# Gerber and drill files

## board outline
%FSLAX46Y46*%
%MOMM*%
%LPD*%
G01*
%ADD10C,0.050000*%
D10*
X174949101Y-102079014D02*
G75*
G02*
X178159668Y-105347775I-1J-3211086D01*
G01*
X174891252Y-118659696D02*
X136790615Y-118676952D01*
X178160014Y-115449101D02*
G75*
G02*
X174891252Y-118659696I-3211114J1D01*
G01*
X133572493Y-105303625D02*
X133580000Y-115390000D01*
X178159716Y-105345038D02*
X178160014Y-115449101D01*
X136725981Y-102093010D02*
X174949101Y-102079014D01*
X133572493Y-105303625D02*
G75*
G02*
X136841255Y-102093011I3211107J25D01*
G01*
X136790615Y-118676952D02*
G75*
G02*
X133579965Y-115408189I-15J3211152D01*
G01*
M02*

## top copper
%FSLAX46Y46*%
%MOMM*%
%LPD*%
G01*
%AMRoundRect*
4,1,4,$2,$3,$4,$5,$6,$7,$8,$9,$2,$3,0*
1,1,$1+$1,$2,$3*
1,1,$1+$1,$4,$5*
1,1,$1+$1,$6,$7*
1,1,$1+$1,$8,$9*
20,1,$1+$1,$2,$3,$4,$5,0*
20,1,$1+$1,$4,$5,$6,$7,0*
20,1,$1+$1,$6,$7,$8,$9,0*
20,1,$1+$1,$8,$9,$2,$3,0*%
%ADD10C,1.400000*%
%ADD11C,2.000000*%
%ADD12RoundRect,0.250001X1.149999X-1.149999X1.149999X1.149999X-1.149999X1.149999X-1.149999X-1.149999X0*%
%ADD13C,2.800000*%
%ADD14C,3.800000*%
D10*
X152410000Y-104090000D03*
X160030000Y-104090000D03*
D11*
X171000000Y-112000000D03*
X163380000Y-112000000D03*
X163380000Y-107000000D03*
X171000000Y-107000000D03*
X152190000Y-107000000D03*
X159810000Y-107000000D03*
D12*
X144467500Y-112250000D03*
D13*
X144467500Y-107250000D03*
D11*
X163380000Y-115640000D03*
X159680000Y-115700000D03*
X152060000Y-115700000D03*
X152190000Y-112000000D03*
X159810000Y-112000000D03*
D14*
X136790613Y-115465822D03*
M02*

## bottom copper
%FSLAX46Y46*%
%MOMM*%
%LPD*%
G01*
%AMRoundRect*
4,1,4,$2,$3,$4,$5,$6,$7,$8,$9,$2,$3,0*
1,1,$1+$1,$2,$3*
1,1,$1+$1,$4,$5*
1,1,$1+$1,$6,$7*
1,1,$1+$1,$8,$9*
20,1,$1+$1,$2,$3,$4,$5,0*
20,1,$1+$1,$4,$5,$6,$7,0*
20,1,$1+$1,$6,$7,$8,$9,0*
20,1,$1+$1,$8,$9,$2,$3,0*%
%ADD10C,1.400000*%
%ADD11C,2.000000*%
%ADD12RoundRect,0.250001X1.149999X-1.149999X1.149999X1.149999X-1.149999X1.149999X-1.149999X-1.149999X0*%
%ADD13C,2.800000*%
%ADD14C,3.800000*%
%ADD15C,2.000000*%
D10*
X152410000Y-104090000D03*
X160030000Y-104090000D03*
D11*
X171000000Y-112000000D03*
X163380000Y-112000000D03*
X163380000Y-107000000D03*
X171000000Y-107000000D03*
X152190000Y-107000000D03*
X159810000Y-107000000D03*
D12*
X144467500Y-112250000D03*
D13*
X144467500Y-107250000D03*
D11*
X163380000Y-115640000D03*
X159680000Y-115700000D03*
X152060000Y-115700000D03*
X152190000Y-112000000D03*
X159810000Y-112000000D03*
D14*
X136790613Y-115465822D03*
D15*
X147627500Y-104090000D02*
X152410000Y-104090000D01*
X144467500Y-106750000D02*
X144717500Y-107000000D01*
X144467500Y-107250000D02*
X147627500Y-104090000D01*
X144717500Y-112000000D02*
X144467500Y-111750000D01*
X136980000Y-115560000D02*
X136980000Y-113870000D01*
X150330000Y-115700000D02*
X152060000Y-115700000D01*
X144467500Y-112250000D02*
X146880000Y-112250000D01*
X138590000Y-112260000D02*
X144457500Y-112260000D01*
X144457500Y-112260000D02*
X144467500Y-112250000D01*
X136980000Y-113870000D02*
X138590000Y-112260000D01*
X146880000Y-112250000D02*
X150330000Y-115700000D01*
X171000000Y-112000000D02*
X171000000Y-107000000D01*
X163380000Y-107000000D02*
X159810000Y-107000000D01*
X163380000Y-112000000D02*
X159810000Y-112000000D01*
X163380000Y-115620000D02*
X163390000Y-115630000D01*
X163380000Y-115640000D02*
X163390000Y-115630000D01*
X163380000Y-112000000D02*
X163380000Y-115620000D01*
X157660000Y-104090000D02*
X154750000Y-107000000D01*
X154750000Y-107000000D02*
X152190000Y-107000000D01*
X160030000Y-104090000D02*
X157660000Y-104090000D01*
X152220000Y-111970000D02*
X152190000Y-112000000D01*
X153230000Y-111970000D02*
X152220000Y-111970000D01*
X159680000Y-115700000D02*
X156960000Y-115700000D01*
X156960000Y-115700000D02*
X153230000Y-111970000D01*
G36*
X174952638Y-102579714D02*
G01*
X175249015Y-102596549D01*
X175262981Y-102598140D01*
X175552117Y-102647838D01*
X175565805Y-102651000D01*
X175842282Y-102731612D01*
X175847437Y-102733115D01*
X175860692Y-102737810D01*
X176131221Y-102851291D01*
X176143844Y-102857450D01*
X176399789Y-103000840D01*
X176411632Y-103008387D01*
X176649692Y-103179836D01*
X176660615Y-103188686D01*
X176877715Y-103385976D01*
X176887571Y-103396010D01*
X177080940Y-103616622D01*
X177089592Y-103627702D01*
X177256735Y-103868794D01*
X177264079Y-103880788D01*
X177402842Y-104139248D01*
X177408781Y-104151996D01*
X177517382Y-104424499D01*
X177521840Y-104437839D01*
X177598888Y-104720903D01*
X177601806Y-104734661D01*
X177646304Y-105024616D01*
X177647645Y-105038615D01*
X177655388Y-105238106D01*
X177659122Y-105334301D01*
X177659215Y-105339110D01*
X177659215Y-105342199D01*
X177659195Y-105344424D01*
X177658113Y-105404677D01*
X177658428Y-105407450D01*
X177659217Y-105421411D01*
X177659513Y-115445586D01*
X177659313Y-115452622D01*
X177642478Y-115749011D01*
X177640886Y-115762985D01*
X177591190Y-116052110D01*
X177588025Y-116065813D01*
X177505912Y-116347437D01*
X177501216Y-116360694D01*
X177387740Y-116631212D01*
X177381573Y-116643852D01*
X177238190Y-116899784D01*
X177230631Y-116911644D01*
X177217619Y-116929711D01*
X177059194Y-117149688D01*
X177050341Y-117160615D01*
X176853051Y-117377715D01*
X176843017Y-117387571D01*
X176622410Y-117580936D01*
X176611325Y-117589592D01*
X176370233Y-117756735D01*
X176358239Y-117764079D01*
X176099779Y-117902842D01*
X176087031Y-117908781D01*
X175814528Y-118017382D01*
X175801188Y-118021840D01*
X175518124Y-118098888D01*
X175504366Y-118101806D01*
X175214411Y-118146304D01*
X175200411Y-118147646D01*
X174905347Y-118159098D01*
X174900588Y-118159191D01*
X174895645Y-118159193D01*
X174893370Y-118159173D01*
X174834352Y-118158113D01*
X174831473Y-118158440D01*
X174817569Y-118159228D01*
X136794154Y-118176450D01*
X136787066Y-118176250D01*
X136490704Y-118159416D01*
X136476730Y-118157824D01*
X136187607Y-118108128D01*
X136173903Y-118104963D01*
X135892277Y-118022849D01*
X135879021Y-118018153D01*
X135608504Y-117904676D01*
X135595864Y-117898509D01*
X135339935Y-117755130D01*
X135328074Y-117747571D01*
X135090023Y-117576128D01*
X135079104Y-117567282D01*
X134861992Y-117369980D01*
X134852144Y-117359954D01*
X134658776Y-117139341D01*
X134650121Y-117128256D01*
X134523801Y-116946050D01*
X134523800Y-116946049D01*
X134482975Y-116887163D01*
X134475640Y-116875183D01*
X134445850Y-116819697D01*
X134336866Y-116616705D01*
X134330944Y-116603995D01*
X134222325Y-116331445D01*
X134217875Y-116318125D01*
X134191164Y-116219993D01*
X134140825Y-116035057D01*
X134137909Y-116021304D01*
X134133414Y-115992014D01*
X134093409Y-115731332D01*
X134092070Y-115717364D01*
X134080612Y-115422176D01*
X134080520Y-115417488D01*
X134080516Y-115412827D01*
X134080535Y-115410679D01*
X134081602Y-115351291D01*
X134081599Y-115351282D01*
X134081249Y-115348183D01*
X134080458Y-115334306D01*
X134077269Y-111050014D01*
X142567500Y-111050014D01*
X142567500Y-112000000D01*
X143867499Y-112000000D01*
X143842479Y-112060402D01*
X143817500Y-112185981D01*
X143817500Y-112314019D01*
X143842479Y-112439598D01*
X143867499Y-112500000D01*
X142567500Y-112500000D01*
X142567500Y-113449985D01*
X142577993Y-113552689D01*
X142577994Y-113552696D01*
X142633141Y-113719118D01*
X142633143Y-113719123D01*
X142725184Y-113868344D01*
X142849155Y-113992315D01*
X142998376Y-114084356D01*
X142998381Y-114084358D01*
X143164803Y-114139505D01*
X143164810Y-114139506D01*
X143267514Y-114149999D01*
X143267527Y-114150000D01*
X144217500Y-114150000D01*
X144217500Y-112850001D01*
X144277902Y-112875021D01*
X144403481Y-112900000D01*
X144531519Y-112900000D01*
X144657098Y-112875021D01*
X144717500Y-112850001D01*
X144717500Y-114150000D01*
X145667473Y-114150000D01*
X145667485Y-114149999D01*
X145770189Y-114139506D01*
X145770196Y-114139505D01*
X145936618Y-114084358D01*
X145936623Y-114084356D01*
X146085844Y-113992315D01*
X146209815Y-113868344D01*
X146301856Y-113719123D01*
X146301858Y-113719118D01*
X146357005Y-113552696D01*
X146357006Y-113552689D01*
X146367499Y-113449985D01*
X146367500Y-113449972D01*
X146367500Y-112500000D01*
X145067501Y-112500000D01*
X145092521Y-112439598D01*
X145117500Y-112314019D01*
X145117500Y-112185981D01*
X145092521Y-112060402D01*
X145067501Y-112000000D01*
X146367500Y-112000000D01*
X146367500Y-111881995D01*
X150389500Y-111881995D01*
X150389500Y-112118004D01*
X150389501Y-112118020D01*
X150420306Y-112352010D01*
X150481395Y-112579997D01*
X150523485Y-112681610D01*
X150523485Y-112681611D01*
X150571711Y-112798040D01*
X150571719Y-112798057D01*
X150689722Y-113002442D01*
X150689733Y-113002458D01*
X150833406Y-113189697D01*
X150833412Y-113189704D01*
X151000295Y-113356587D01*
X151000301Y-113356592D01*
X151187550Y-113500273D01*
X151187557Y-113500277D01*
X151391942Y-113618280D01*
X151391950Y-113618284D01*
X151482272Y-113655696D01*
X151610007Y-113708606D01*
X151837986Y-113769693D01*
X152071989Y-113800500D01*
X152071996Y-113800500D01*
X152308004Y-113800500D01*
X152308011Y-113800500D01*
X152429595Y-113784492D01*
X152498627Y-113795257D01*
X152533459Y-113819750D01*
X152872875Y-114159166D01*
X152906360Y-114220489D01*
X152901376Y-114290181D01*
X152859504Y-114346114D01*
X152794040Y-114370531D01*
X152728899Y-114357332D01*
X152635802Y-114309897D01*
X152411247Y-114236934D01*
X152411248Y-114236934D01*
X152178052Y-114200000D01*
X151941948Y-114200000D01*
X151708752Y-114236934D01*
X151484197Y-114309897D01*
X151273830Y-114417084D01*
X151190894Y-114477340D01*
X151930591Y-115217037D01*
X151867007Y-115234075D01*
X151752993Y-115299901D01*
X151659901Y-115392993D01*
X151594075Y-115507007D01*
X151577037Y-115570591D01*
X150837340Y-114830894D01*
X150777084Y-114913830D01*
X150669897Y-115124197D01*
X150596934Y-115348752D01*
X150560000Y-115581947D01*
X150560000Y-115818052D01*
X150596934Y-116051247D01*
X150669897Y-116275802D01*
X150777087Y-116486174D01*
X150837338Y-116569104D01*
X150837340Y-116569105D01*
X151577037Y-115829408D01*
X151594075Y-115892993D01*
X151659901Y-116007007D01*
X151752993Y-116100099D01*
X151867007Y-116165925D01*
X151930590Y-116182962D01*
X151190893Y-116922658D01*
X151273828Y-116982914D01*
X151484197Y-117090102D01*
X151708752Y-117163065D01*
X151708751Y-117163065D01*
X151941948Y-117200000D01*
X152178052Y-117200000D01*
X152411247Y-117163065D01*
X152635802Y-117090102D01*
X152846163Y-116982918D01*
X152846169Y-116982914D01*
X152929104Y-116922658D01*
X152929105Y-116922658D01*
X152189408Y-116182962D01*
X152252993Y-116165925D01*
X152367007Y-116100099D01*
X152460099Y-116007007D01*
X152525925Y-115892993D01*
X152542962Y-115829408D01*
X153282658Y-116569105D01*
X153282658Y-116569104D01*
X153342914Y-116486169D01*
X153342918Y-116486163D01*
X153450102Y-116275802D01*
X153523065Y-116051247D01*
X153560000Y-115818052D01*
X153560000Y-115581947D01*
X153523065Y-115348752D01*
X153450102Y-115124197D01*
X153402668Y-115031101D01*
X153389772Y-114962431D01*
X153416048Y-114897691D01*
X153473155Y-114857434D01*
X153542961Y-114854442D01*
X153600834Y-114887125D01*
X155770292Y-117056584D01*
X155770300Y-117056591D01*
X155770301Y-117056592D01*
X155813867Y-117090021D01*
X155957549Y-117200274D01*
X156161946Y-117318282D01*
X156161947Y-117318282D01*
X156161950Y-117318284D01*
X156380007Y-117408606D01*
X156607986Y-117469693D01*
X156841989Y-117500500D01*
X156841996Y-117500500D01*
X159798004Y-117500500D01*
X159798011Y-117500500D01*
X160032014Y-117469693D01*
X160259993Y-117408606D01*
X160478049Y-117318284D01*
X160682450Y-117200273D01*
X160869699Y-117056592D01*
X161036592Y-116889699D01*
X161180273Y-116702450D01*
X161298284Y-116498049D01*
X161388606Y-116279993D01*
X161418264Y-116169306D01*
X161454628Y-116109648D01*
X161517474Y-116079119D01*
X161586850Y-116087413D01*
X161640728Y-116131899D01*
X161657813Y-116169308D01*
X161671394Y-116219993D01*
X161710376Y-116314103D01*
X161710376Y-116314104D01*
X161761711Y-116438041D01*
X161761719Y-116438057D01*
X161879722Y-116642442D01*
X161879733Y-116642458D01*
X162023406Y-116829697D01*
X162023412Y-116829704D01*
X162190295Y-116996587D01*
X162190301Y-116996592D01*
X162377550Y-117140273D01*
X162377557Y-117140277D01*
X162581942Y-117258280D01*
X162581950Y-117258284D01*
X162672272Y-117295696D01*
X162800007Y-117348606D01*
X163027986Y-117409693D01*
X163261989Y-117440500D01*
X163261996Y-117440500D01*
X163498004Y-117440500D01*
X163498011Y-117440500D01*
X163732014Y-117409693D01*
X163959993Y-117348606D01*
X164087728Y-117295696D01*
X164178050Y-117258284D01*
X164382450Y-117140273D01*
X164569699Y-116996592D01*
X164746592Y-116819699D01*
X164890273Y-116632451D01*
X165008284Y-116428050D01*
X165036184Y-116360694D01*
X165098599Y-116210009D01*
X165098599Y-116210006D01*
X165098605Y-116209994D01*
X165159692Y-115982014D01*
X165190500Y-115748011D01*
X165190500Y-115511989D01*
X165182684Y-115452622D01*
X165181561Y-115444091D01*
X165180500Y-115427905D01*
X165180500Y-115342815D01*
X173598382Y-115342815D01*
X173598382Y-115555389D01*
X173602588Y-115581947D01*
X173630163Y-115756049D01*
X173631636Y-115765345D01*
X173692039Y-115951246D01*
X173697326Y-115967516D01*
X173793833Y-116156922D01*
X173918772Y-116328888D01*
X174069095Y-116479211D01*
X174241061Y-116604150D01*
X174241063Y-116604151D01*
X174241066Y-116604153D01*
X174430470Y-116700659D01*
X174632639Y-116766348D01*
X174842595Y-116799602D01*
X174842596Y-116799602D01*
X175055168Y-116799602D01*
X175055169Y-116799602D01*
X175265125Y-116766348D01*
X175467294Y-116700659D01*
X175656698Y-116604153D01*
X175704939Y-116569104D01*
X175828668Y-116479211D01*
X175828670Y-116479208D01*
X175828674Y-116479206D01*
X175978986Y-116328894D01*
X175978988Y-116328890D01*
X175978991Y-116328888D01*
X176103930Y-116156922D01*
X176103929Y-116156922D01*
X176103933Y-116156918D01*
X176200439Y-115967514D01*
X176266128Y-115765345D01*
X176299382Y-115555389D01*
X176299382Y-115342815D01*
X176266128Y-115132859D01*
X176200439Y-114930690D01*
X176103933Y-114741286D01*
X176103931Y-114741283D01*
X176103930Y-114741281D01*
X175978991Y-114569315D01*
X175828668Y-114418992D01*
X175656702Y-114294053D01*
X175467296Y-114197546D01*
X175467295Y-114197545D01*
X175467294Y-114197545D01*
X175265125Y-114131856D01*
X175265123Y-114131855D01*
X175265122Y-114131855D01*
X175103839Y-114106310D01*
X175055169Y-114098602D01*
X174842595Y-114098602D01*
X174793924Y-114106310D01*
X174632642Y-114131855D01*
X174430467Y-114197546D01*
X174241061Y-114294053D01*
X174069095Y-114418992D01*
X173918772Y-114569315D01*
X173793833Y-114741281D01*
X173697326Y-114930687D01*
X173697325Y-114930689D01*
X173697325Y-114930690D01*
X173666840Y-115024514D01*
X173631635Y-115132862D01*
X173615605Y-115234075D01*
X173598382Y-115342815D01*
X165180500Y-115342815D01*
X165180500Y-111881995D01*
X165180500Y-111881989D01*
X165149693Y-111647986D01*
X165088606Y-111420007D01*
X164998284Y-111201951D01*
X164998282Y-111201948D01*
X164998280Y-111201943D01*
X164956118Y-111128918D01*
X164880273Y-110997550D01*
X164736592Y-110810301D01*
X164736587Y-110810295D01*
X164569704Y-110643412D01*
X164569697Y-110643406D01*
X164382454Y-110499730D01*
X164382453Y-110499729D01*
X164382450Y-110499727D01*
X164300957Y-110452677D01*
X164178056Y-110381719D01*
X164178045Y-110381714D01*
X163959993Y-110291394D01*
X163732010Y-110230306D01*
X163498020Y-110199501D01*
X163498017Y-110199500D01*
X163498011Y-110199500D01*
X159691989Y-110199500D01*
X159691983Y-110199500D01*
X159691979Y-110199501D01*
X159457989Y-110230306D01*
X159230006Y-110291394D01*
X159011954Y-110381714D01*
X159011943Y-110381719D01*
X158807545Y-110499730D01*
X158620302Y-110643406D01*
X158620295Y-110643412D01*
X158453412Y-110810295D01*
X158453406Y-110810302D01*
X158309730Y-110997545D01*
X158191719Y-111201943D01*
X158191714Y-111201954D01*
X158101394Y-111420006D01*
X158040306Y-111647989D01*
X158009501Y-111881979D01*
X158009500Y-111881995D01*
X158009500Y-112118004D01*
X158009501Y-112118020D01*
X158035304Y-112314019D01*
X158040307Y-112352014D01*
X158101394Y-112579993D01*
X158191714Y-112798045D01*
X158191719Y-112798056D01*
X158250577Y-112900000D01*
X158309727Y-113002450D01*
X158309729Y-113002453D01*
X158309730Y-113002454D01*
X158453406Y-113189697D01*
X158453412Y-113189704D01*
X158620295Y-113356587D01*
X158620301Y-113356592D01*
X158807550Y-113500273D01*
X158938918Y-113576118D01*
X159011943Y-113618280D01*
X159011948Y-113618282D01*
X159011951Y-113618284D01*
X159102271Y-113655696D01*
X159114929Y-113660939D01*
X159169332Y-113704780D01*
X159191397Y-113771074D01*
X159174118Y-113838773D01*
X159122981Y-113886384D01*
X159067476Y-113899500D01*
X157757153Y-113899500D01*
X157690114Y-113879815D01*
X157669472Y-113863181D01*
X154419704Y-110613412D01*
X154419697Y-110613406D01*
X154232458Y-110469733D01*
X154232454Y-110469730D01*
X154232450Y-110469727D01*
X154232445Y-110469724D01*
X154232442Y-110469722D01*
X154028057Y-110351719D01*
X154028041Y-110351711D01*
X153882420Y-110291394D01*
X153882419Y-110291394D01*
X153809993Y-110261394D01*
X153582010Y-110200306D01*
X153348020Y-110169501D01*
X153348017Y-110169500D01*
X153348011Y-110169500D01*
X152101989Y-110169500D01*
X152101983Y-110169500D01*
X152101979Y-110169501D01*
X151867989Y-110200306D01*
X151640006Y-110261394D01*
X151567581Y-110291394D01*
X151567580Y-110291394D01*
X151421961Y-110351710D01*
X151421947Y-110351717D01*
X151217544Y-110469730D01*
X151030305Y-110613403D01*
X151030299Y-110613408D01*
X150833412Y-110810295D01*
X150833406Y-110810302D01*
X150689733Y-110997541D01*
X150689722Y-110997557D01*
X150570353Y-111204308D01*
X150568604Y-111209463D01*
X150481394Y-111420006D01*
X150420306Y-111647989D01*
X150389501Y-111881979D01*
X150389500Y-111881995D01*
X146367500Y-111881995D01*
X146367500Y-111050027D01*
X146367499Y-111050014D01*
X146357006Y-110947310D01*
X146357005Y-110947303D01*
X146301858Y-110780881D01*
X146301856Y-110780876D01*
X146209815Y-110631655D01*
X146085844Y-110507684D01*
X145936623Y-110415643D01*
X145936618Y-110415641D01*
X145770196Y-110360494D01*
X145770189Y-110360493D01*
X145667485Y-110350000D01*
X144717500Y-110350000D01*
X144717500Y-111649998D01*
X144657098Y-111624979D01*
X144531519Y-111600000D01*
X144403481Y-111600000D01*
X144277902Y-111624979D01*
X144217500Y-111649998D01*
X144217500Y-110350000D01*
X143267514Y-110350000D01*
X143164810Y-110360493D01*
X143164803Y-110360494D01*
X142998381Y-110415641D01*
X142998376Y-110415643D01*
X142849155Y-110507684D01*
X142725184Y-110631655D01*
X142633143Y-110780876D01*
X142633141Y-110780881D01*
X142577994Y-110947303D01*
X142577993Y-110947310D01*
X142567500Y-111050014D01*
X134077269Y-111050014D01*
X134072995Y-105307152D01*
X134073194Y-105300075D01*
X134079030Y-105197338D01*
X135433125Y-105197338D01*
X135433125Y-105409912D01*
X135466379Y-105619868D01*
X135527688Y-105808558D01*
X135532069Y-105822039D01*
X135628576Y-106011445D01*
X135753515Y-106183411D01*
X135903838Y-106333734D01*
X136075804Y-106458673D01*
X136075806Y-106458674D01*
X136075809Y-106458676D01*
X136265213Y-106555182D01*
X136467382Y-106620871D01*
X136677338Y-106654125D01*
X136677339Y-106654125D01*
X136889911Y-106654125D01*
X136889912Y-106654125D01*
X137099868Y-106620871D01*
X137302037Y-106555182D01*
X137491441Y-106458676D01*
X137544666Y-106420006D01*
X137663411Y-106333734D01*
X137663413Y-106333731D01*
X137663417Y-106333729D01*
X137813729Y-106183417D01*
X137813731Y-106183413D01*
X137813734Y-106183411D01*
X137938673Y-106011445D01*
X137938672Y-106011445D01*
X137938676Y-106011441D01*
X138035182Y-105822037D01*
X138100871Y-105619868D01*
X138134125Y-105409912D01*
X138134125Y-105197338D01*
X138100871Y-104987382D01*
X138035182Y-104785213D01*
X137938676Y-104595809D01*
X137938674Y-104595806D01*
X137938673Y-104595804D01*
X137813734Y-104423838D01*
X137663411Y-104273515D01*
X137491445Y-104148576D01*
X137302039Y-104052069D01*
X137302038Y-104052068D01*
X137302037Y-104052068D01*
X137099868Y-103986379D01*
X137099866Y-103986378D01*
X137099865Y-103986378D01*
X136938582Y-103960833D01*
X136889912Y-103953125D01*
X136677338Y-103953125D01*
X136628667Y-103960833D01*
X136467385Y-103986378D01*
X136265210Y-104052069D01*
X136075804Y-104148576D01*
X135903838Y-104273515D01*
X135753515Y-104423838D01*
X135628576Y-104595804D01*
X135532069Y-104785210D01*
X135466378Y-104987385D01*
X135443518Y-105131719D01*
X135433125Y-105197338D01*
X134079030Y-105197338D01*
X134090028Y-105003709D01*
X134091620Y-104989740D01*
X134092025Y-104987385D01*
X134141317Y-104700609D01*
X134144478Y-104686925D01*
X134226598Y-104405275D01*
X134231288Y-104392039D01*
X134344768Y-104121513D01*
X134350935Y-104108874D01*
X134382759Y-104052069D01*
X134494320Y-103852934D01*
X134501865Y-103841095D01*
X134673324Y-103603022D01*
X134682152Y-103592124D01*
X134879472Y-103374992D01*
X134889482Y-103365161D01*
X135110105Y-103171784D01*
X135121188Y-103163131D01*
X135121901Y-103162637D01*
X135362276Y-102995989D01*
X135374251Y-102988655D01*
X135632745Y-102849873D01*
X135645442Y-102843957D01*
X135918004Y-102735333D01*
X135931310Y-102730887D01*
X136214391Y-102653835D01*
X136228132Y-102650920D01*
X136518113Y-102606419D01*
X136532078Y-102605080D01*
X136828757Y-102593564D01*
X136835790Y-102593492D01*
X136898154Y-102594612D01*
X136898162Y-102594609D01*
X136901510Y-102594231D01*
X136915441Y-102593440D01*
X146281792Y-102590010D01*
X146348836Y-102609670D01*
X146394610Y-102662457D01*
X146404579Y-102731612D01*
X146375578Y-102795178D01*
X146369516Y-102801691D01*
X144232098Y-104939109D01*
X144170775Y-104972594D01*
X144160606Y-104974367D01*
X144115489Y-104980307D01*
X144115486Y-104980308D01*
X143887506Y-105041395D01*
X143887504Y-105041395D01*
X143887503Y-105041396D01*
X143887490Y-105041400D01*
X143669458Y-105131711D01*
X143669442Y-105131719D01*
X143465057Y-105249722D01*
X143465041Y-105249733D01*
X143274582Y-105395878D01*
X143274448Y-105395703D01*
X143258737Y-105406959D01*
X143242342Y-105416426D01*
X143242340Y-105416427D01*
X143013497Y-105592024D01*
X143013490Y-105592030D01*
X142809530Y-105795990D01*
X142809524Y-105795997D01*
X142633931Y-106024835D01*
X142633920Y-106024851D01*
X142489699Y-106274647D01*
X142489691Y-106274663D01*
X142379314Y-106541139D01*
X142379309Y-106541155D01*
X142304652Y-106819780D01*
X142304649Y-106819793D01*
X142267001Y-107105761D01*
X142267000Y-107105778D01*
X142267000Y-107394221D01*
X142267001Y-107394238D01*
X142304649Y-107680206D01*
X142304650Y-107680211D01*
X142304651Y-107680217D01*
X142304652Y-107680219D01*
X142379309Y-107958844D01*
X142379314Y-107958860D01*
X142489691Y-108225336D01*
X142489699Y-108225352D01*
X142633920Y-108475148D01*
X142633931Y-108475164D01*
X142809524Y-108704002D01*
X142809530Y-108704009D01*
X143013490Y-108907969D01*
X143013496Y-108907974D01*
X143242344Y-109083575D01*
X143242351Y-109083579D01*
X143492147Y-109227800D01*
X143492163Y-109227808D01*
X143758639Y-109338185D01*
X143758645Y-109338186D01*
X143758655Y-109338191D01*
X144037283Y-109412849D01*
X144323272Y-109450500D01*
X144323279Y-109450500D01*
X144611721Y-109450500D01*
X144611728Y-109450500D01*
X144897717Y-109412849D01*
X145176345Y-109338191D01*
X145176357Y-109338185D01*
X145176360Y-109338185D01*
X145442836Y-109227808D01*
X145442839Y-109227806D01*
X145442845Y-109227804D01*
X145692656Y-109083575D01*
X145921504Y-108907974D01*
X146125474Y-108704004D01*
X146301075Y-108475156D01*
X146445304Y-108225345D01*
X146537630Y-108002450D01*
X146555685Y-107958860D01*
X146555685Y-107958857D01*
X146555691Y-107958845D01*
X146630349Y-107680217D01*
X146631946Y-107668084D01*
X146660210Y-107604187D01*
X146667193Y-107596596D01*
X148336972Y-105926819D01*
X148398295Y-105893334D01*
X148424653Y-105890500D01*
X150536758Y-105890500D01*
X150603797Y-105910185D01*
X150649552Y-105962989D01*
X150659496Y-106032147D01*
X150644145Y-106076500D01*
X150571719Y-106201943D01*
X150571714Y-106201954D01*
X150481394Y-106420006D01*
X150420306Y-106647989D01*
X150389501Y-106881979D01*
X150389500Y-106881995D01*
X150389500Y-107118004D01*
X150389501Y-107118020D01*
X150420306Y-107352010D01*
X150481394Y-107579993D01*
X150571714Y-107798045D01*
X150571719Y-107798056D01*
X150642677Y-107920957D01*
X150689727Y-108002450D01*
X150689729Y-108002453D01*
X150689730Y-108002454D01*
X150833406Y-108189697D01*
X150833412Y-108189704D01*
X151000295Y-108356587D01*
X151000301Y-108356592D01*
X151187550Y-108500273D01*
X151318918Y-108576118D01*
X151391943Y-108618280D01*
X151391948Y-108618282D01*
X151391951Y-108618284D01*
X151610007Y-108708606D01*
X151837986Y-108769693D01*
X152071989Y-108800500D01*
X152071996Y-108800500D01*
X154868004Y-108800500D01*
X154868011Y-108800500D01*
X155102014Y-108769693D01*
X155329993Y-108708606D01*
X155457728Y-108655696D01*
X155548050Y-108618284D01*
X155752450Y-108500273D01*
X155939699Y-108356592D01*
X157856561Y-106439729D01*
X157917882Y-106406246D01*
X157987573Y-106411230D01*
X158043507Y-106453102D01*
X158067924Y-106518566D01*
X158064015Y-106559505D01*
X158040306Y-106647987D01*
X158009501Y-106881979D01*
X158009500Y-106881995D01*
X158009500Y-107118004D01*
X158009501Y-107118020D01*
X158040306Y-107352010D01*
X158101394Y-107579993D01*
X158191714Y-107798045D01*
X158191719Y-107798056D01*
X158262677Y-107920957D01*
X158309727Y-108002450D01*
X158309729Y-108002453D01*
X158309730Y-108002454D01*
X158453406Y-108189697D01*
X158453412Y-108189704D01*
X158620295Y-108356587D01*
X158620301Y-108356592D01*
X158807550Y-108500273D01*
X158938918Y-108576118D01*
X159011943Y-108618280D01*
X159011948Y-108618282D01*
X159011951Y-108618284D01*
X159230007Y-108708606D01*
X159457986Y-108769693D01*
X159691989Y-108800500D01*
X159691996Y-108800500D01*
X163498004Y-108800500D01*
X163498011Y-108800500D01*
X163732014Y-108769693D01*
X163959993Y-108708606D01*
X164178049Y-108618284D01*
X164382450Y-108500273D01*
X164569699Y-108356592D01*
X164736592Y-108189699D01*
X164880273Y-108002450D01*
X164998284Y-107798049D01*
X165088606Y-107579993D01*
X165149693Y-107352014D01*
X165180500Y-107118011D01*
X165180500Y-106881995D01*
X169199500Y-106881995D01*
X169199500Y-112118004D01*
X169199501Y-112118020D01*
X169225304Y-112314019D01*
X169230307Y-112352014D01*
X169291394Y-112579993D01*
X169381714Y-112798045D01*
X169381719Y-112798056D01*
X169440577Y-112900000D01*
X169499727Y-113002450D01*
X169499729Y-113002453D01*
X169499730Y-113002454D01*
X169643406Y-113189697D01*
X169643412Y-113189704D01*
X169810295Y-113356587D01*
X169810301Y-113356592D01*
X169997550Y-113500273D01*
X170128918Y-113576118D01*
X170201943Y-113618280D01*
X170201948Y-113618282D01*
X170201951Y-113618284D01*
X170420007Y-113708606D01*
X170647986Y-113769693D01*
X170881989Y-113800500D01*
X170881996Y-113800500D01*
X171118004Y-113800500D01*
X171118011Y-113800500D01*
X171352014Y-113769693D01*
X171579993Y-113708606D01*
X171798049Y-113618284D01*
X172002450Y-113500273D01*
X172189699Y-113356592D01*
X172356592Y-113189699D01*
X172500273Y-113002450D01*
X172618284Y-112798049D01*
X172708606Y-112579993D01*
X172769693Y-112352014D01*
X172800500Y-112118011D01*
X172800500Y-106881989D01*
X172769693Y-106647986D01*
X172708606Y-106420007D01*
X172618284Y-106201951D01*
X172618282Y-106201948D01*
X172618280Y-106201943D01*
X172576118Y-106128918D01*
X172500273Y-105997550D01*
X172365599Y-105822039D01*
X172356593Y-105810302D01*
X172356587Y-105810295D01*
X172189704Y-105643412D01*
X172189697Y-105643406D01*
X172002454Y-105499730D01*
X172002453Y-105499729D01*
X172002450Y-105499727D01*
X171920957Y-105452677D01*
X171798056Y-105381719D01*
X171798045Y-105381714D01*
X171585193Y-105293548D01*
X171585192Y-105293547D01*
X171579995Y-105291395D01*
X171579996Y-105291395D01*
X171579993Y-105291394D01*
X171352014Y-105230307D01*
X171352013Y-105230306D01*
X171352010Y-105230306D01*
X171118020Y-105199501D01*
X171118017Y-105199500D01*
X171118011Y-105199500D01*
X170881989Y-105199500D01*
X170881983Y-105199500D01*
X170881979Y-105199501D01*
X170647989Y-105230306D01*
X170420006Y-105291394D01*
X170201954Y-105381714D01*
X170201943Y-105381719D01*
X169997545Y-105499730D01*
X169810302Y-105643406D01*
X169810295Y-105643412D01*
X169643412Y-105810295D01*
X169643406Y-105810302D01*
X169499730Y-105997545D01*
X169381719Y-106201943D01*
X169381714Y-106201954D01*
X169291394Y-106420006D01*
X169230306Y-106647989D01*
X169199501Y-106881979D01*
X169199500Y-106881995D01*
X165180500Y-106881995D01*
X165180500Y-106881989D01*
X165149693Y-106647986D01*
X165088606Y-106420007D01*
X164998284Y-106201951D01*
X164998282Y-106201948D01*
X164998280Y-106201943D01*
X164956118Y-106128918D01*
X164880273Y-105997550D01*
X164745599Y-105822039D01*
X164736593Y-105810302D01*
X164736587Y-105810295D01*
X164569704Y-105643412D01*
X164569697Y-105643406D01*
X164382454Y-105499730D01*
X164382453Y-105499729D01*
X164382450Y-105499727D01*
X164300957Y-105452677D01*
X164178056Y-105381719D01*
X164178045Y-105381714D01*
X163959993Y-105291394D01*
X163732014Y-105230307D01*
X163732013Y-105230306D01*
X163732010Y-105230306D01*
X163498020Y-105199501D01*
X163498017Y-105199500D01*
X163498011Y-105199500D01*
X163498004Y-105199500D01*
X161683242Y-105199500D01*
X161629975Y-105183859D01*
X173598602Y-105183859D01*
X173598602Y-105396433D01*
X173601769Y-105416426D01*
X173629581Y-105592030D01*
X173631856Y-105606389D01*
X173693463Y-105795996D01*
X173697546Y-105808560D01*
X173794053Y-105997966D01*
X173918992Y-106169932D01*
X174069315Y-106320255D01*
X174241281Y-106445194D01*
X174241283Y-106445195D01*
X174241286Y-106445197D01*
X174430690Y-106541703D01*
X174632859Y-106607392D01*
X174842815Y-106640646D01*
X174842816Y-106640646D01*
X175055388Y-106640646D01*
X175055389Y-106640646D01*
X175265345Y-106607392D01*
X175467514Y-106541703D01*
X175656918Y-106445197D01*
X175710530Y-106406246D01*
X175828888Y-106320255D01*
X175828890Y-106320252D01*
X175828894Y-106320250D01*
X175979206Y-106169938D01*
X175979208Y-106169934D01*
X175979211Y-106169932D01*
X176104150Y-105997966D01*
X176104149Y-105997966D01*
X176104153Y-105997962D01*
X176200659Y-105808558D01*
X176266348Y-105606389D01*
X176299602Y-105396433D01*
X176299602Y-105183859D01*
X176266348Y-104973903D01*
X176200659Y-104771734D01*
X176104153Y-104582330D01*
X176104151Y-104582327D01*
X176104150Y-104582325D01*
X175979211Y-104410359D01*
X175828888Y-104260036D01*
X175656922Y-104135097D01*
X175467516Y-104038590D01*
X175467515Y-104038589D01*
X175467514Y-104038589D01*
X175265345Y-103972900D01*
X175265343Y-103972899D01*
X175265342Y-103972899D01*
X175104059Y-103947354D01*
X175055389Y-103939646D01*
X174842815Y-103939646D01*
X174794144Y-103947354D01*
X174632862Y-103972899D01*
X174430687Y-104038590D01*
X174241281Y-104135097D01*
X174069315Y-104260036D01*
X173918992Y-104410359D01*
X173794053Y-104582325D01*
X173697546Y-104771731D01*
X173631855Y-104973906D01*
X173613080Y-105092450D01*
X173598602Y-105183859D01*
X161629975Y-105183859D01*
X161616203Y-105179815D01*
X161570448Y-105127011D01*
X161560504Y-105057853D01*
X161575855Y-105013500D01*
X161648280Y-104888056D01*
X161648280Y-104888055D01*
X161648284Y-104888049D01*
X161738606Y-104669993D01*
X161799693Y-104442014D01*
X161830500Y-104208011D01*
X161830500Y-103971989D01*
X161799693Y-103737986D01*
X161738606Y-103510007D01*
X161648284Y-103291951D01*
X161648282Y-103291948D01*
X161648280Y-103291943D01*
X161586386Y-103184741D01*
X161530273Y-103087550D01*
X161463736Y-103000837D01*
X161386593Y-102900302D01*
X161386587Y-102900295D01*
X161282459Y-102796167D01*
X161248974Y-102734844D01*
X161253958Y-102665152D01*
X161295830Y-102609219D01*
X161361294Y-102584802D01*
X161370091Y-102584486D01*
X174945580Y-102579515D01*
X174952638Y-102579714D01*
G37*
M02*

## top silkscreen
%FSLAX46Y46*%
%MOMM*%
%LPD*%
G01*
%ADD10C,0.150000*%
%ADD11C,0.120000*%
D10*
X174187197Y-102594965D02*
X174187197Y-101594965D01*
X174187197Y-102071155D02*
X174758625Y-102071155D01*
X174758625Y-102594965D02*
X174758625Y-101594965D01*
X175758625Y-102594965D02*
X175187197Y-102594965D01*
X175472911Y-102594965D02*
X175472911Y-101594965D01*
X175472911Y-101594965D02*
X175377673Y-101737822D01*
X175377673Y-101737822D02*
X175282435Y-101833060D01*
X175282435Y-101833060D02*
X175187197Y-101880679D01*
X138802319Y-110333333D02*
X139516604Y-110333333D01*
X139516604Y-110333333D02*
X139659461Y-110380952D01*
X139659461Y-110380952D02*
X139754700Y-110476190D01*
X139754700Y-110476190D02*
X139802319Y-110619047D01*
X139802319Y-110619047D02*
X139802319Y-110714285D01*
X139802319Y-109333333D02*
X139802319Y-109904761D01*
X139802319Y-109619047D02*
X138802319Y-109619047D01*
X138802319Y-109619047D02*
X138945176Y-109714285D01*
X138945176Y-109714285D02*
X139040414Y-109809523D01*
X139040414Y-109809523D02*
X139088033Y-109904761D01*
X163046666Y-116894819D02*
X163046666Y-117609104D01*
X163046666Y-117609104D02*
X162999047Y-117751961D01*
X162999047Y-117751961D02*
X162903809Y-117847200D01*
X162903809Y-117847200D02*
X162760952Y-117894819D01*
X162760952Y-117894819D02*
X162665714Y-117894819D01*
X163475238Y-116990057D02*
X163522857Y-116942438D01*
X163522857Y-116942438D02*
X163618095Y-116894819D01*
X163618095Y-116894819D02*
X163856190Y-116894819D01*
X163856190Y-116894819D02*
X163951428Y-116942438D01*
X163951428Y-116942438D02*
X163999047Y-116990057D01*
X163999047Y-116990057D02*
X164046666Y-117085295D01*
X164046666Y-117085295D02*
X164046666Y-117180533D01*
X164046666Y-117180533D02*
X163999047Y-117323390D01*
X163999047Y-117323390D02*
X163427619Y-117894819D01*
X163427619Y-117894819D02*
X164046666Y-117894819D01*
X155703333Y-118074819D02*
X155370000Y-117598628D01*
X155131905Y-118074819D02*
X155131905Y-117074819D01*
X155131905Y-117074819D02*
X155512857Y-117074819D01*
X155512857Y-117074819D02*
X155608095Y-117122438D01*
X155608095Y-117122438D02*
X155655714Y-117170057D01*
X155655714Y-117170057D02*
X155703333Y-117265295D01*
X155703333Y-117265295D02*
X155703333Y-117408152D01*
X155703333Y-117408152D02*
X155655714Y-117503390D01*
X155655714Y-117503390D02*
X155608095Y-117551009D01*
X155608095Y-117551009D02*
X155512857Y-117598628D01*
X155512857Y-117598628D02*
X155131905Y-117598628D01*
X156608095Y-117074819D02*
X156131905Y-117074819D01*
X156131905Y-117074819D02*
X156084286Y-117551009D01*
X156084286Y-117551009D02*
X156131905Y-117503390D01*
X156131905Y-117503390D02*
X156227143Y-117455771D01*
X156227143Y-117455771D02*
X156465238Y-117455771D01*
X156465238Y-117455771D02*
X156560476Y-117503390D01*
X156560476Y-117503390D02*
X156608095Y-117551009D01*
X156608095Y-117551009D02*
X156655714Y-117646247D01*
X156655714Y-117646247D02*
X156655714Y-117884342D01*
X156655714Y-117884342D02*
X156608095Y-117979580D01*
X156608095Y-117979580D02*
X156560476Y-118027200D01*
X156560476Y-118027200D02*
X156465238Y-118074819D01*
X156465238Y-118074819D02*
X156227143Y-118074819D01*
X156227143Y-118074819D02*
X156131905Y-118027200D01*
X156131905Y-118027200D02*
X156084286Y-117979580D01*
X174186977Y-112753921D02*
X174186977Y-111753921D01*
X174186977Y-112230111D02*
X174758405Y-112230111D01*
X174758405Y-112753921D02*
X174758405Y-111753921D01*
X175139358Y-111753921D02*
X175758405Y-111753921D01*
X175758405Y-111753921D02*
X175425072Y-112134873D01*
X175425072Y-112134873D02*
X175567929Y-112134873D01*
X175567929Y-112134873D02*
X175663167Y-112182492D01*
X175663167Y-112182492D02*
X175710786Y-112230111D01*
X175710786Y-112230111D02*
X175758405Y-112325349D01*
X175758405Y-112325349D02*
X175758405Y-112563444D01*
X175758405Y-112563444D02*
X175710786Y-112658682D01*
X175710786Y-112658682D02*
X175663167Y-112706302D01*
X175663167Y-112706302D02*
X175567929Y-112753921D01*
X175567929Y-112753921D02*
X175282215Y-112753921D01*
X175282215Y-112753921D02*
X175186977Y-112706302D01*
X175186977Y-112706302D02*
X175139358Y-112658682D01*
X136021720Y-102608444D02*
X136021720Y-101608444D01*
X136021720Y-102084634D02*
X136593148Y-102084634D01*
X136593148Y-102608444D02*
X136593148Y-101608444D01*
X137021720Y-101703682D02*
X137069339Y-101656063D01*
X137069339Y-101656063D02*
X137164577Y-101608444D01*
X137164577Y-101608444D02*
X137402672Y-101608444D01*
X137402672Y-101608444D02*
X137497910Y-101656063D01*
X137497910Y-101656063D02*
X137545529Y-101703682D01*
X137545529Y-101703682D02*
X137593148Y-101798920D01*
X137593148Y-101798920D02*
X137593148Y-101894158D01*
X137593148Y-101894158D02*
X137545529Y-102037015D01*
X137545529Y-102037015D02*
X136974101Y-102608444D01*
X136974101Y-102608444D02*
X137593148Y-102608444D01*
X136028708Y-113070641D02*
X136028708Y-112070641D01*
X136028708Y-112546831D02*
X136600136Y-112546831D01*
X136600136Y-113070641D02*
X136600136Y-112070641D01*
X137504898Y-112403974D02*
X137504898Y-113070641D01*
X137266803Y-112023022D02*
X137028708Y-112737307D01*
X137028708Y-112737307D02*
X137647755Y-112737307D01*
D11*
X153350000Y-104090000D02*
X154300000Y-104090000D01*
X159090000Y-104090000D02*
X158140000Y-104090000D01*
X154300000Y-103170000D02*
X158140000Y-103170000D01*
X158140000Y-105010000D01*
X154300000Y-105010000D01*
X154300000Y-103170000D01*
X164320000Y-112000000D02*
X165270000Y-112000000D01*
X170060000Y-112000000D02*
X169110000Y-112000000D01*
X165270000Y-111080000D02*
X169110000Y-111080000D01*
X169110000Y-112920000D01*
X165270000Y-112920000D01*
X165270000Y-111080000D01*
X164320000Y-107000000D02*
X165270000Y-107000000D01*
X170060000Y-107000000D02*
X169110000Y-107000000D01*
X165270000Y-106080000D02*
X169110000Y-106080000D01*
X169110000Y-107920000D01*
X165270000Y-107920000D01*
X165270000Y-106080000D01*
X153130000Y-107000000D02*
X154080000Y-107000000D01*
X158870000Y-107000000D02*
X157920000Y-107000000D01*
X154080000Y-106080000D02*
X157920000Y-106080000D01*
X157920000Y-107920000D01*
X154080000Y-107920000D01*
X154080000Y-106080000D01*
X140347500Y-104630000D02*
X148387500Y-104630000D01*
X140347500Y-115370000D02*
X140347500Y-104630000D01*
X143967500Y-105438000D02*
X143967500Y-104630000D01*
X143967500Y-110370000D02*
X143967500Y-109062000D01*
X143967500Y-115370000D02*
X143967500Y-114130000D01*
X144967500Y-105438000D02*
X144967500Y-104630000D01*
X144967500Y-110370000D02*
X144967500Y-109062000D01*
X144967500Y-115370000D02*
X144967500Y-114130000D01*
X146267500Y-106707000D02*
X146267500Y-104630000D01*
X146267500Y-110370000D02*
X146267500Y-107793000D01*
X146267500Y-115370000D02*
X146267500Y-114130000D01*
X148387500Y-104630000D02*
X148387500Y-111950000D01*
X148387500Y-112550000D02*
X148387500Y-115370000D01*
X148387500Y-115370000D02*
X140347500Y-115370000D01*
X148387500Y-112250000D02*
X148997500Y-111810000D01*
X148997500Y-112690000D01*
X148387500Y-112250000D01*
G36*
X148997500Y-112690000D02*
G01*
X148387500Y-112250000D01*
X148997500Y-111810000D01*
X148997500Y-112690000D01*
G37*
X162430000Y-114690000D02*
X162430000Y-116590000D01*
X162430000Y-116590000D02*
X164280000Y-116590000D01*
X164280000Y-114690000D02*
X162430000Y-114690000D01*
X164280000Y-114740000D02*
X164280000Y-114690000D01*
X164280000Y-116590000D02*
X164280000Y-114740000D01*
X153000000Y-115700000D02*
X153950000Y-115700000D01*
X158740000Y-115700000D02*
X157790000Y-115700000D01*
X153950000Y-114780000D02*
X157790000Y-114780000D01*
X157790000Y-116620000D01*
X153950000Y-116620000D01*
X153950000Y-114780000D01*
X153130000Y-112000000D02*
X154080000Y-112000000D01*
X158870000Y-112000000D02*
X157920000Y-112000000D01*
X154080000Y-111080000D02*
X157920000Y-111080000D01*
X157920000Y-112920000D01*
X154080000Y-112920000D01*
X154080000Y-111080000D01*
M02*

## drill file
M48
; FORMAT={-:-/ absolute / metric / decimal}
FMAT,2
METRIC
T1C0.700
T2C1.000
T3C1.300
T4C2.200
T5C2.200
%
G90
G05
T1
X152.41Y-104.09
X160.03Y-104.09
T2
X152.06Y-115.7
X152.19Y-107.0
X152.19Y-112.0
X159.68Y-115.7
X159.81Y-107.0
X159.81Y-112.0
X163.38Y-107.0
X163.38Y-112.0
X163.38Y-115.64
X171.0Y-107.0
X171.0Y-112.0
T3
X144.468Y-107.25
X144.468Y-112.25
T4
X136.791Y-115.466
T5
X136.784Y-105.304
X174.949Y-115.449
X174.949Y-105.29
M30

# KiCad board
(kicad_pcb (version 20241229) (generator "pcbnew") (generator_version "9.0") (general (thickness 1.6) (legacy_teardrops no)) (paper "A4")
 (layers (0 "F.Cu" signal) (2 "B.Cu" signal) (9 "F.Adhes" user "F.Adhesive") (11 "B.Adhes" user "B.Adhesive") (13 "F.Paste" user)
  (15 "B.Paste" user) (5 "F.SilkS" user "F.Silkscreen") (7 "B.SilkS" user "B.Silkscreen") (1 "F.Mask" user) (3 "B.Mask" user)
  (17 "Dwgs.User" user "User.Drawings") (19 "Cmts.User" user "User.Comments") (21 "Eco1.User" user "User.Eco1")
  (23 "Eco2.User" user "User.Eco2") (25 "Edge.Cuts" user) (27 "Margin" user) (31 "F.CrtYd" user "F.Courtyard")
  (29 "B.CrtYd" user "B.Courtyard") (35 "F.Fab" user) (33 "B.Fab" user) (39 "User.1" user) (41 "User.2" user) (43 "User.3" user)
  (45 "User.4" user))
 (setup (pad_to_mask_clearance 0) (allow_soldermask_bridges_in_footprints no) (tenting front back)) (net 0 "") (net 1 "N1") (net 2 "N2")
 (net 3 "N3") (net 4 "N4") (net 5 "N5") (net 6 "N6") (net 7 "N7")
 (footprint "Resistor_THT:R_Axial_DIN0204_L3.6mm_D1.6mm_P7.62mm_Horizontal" (layer "F.Cu") (at 152.41 104.09)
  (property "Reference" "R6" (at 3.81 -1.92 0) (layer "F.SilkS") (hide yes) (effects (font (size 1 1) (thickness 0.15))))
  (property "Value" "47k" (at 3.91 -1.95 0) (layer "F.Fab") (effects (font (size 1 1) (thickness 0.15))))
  (fp_line (start 0.94 0) (end 1.89 0) (stroke (width 0.12) (type solid)) (layer "F.SilkS"))
  (fp_line (start 6.68 0) (end 5.73 0) (stroke (width 0.12) (type solid)) (layer "F.SilkS"))
  (fp_rect (start 1.89 -0.92) (end 5.73 0.92) (stroke (width 0.12) (type solid)) (fill no) (layer "F.SilkS"))
  (pad "1" thru_hole circle (at 0 0) (size 1.4 1.4) (drill 0.7) (layers "*.Cu" "*.Mask") (remove_unused_layers no) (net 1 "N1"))
  (pad "2" thru_hole circle (at 7.62 0) (size 1.4 1.4) (drill 0.7) (layers "*.Cu" "*.Mask") (remove_unused_layers no) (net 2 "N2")))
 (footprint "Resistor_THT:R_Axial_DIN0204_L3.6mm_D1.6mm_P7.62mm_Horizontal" (layer "F.Cu") (at 171 112 180)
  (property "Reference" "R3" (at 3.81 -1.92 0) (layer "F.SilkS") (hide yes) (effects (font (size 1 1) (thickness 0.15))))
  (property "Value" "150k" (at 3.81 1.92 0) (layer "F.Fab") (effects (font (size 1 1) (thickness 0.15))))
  (fp_line (start 6.68 0) (end 5.73 0) (stroke (width 0.12) (type solid)) (layer "F.SilkS"))
  (fp_line (start 0.94 0) (end 1.89 0) (stroke (width 0.12) (type solid)) (layer "F.SilkS"))
  (fp_rect (start 1.89 -0.92) (end 5.73 0.92) (stroke (width 0.12) (type solid)) (fill no) (layer "F.SilkS"))
  (pad "1" thru_hole circle (at 0 0 180) (size 2 2) (drill 1) (layers "*.Cu" "*.Mask") (remove_unused_layers no) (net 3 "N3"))
  (pad "2" thru_hole circle (at 7.62 0 180) (size 2 2) (drill 1) (layers "*.Cu" "*.Mask") (remove_unused_layers no) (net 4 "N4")))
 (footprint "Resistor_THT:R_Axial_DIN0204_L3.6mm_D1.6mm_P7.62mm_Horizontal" (layer "F.Cu") (at 163.38 107)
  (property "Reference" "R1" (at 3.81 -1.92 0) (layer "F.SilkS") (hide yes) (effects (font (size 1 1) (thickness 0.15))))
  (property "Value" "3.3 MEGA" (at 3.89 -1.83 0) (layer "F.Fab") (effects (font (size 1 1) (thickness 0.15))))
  (fp_line (start 0.94 0) (end 1.89 0) (stroke (width 0.12) (type solid)) (layer "F.SilkS"))
  (fp_line (start 6.68 0) (end 5.73 0) (stroke (width 0.12) (type solid)) (layer "F.SilkS"))
  (fp_rect (start 1.89 -0.92) (end 5.73 0.92) (stroke (width 0.12) (type solid)) (fill no) (layer "F.SilkS"))
  (pad "1" thru_hole circle (at 0 0) (size 2 2) (drill 1) (layers "*.Cu" "*.Mask") (remove_unused_layers no) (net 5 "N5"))
  (pad "2" thru_hole circle (at 7.62 0) (size 2 2) (drill 1) (layers "*.Cu" "*.Mask") (remove_unused_layers no) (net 3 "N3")))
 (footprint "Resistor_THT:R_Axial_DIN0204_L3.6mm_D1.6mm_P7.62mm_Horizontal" (layer "F.Cu") (at 152.19 107)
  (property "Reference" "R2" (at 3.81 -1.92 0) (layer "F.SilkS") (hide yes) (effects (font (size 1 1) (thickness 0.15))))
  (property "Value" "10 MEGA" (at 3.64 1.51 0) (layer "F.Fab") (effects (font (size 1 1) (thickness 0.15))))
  (fp_line (start 0.94 0) (end 1.89 0) (stroke (width 0.12) (type solid)) (layer "F.SilkS"))
  (fp_line (start 6.68 0) (end 5.73 0) (stroke (width 0.12) (type solid)) (layer "F.SilkS"))
  (fp_rect (start 1.89 -0.92) (end 5.73 0.92) (stroke (width 0.12) (type solid)) (fill no) (layer "F.SilkS"))
  (pad "1" thru_hole circle (at 0 0) (size 2 2) (drill 1) (layers "*.Cu" "*.Mask") (remove_unused_layers no) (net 2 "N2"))
  (pad "2" thru_hole circle (at 7.62 0) (size 2 2) (drill 1) (layers "*.Cu" "*.Mask") (remove_unused_layers no) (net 5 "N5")))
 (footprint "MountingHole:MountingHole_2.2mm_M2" (layer "F.Cu") (at 174.949102 105.290146)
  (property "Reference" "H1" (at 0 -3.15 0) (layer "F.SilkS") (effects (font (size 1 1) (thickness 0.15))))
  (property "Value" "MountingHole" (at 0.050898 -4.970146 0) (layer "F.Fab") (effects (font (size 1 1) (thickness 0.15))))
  (pad "" np_thru_hole circle (at 0 0) (size 2.2 2.2) (drill 2.2) (layers "*.Cu" "*.Mask")))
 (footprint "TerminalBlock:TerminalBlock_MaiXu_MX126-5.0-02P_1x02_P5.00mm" (layer "F.Cu") (at 144.4675 112.25 90)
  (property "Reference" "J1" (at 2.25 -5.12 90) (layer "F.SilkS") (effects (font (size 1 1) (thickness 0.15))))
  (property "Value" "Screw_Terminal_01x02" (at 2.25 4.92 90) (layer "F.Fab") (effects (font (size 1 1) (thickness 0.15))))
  (fp_line (start 7.62 -4.12) (end 7.62 3.92) (stroke (width 0.12) (type solid)) (layer "F.SilkS"))
  (fp_line (start -3.12 -4.12) (end 7.62 -4.12) (stroke (width 0.12) (type solid)) (layer "F.SilkS"))
  (fp_line (start 6.812 -0.5) (end 7.62 -0.5) (stroke (width 0.12) (type solid)) (layer "F.SilkS"))
  (fp_line (start 1.88 -0.5) (end 3.188 -0.5) (stroke (width 0.12) (type solid)) (layer "F.SilkS"))
  (fp_line (start -3.12 -0.5) (end -1.88 -0.5) (stroke (width 0.12) (type solid)) (layer "F.SilkS"))
  (fp_line (start 6.812 0.5) (end 7.62 0.5) (stroke (width 0.12) (type solid)) (layer "F.SilkS"))
  (fp_line (start 1.88 0.5) (end 3.188 0.5) (stroke (width 0.12) (type solid)) (layer "F.SilkS"))
  (fp_line (start -3.12 0.5) (end -1.88 0.5) (stroke (width 0.12) (type solid)) (layer "F.SilkS"))
  (fp_line (start 5.543 1.8) (end 7.62 1.8) (stroke (width 0.12) (type solid)) (layer "F.SilkS"))
  (fp_line (start 1.88 1.8) (end 4.457 1.8) (stroke (width 0.12) (type solid)) (layer "F.SilkS"))
  (fp_line (start -3.12 1.8) (end -1.88 1.8) (stroke (width 0.12) (type solid)) (layer "F.SilkS"))
  (fp_line (start 7.62 3.92) (end 0.3 3.92) (stroke (width 0.12) (type solid)) (layer "F.SilkS"))
  (fp_line (start -0.3 3.92) (end -3.12 3.92) (stroke (width 0.12) (type solid)) (layer "F.SilkS"))
  (fp_line (start -3.12 3.92) (end -3.12 -4.12) (stroke (width 0.12) (type solid)) (layer "F.SilkS"))
  (fp_poly (pts (xy 0 3.92) (xy 0.44 4.53) (xy -0.44 4.53)) (stroke (width 0.12) (type solid)) (fill yes) (layer "F.SilkS"))
  (pad "1" thru_hole roundrect (at 0 0 90) (size 2.8 2.8) (drill 1.3) (layers "*.Cu" "*.Mask") (remove_unused_layers no)
   (roundrect_rratio 0.089286) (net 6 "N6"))
  (pad "2" thru_hole circle (at 5 0 90) (size 2.8 2.8) (drill 1.3) (layers "*.Cu" "*.Mask") (remove_unused_layers no) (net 1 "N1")))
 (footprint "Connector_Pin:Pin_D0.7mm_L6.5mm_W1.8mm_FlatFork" (layer "F.Cu") (at 163.38 115.64)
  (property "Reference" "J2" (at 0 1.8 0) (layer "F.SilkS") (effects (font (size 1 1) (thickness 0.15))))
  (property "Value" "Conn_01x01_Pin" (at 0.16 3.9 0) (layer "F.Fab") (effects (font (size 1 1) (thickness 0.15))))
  (fp_line (start -0.95 -0.95) (end -0.95 0.95) (stroke (width 0.12) (type solid)) (layer "F.SilkS"))
  (fp_line (start -0.95 0.95) (end 0.9 0.95) (stroke (width 0.12) (type solid)) (layer "F.SilkS"))
  (fp_line (start 0.9 -0.95) (end -0.95 -0.95) (stroke (width 0.12) (type solid)) (layer "F.SilkS"))
  (fp_line (start 0.9 -0.9) (end 0.9 -0.95) (stroke (width 0.12) (type solid)) (layer "F.SilkS"))
  (fp_line (start 0.9 0.95) (end 0.9 -0.9) (stroke (width 0.12) (type solid)) (layer "F.SilkS"))
  (pad "1" thru_hole circle (at 0 0) (size 2 2) (drill 1) (layers "*.Cu" "*.Mask") (remove_unused_layers no) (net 4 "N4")))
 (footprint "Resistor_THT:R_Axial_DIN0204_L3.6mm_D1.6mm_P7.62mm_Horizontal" (layer "F.Cu") (at 159.68 115.7 180)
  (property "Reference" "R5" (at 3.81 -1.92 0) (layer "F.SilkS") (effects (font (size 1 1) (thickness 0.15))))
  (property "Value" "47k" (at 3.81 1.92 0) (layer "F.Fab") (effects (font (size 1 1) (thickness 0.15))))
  (fp_line (start 6.68 0) (end 5.73 0) (stroke (width 0.12) (type solid)) (layer "F.SilkS"))
  (fp_line (start 0.94 0) (end 1.89 0) (stroke (width 0.12) (type solid)) (layer "F.SilkS"))
  (fp_rect (start 1.89 -0.92) (end 5.73 0.92) (stroke (width 0.12) (type solid)) (fill no) (layer "F.SilkS"))
  (pad "1" thru_hole circle (at 0 0 180) (size 2 2) (drill 1) (layers "*.Cu" "*.Mask") (remove_unused_layers no) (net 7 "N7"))
  (pad "2" thru_hole circle (at 7.62 0 180) (size 2 2) (drill 1) (layers "*.Cu" "*.Mask") (remove_unused_layers no) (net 6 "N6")))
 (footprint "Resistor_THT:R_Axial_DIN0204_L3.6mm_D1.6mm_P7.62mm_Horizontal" (layer "F.Cu") (at 152.19 112)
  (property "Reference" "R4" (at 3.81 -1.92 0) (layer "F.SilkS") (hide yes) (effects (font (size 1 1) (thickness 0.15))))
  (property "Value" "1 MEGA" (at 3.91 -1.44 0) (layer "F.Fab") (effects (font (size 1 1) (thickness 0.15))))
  (fp_line (start 0.94 0) (end 1.89 0) (stroke (width 0.12) (type solid)) (layer "F.SilkS"))
  (fp_line (start 6.68 0) (end 5.73 0) (stroke (width 0.12) (type solid)) (layer "F.SilkS"))
  (fp_rect (start 1.89 -0.92) (end 5.73 0.92) (stroke (width 0.12) (type solid)) (fill no) (layer "F.SilkS"))
  (pad "1" thru_hole circle (at 0 0) (size 2 2) (drill 1) (layers "*.Cu" "*.Mask") (remove_unused_layers no) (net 7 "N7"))
  (pad "2" thru_hole circle (at 7.62 0) (size 2 2) (drill 1) (layers "*.Cu" "*.Mask") (remove_unused_layers no) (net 4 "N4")))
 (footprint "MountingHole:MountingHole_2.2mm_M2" (layer "F.Cu") (at 174.948882 115.449102)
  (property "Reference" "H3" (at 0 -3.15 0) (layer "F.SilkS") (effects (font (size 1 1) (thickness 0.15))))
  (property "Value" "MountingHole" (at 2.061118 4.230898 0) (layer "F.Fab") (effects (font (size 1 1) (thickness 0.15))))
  (pad "" np_thru_hole circle (at 0 0) (size 2.2 2.2) (drill 2.2) (layers "*.Cu" "*.Mask")))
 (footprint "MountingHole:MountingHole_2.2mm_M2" (layer "F.Cu") (at 136.783625 105.303625)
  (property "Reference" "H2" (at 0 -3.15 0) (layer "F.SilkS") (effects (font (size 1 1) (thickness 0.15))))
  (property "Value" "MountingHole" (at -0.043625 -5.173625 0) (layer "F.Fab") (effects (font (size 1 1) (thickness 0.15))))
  (pad "" np_thru_hole circle (at 0 0) (size 2.2 2.2) (drill 2.2) (layers "*.Cu" "*.Mask")))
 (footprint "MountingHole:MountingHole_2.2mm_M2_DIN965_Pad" (layer "F.Cu") (at 136.790613 115.465822)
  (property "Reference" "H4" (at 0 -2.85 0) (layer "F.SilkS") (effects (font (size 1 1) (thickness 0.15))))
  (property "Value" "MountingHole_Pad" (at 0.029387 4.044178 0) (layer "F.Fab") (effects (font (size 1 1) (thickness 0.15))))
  (pad "1" thru_hole circle (at 0 0) (size 3.8 3.8) (drill 2.2) (layers "*.Cu" "*.Mask") (remove_unused_layers no) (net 6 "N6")
   (zone_connect 2)))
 (gr_arc (start 174.949101 102.079014) (mid 177.24 103.04) (end 178.159716 105.347776) (stroke (width 0.05) (type default))
  (layer "Edge.Cuts"))
 (gr_line (start 174.891252 118.659696) (end 136.790615 118.676952) (stroke (width 0.05) (type default)) (layer "Edge.Cuts"))
 (gr_arc (start 178.160014 115.449101) (mid 177.199028 117.74) (end 174.891252 118.659716) (stroke (width 0.05) (type default))
  (layer "Edge.Cuts"))
 (gr_line (start 133.572493 105.303625) (end 133.58 115.39) (stroke (width 0.05) (type default)) (layer "Edge.Cuts"))
 (gr_line (start 178.159716 105.345038) (end 178.160014 115.449101) (stroke (width 0.05) (type default)) (layer "Edge.Cuts"))
 (gr_line (start 136.725981 102.09301) (end 174.949101 102.079014) (stroke (width 0.05) (type default)) (layer "Edge.Cuts"))
 (gr_arc (start 133.572493 105.303625) (mid 134.533479 103.012727) (end 136.841255 102.09301) (stroke (width 0.05) (type default))
  (layer "Edge.Cuts"))
 (gr_arc (start 136.790615 118.676952) (mid 134.499717 117.715966) (end 133.58 115.40819) (stroke (width 0.05) (type default))
  (layer "Edge.Cuts"))
 (segment (start 147.6275 104.09) (end 152.41 104.09) (width 2) (layer "B.Cu") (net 1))
 (segment (start 144.4675 106.75) (end 144.7175 107) (width 2) (layer "B.Cu") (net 1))
 (segment (start 144.4675 107.25) (end 147.6275 104.09) (width 2) (layer "B.Cu") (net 1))
 (segment (start 144.7175 112) (end 144.4675 111.75) (width 2) (layer "B.Cu") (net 6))
 (segment (start 136.98 115.56) (end 136.98 113.87) (width 2) (layer "B.Cu") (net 6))
 (segment (start 150.33 115.7) (end 152.06 115.7) (width 2) (layer "B.Cu") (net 6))
 (segment (start 144.4675 112.25) (end 146.88 112.25) (width 2) (layer "B.Cu") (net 6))
 (segment (start 138.59 112.26) (end 144.4575 112.26) (width 2) (layer "B.Cu") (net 6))
 (segment (start 144.4575 112.26) (end 144.4675 112.25) (width 2) (layer "B.Cu") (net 6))
 (segment (start 136.98 113.87) (end 138.59 112.26) (width 2) (layer "B.Cu") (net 6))
 (segment (start 146.88 112.25) (end 150.33 115.7) (width 2) (layer "B.Cu") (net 6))
 (segment (start 171 112) (end 171 107) (width 2) (layer "B.Cu") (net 3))
 (segment (start 163.38 107) (end 159.81 107) (width 2) (layer "B.Cu") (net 5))
 (segment (start 163.38 112) (end 159.81 112) (width 2) (layer "B.Cu") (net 4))
 (segment (start 163.38 115.62) (end 163.39 115.63) (width 2) (layer "B.Cu") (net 4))
 (segment (start 163.38 115.64) (end 163.39 115.63) (width 2) (layer "B.Cu") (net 4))
 (segment (start 163.38 112) (end 163.38 115.62) (width 2) (layer "B.Cu") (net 4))
 (segment (start 157.66 104.09) (end 154.75 107) (width 2) (layer "B.Cu") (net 2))
 (segment (start 154.75 107) (end 152.19 107) (width 2) (layer "B.Cu") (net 2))
 (segment (start 160.03 104.09) (end 157.66 104.09) (width 2) (layer "B.Cu") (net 2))
 (segment (start 152.22 111.97) (end 152.19 112) (width 2) (layer "B.Cu") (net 7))
 (segment (start 153.23 111.97) (end 152.22 111.97) (width 2) (layer "B.Cu") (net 7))
 (segment (start 159.68 115.7) (end 156.96 115.7) (width 2) (layer "B.Cu") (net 7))
 (segment (start 156.96 115.7) (end 153.23 111.97) (width 2) (layer "B.Cu") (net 7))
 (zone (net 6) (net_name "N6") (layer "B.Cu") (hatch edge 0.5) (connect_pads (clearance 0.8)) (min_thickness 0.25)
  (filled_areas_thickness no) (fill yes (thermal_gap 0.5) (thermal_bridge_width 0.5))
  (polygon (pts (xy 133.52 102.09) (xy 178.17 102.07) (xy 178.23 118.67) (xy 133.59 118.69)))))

